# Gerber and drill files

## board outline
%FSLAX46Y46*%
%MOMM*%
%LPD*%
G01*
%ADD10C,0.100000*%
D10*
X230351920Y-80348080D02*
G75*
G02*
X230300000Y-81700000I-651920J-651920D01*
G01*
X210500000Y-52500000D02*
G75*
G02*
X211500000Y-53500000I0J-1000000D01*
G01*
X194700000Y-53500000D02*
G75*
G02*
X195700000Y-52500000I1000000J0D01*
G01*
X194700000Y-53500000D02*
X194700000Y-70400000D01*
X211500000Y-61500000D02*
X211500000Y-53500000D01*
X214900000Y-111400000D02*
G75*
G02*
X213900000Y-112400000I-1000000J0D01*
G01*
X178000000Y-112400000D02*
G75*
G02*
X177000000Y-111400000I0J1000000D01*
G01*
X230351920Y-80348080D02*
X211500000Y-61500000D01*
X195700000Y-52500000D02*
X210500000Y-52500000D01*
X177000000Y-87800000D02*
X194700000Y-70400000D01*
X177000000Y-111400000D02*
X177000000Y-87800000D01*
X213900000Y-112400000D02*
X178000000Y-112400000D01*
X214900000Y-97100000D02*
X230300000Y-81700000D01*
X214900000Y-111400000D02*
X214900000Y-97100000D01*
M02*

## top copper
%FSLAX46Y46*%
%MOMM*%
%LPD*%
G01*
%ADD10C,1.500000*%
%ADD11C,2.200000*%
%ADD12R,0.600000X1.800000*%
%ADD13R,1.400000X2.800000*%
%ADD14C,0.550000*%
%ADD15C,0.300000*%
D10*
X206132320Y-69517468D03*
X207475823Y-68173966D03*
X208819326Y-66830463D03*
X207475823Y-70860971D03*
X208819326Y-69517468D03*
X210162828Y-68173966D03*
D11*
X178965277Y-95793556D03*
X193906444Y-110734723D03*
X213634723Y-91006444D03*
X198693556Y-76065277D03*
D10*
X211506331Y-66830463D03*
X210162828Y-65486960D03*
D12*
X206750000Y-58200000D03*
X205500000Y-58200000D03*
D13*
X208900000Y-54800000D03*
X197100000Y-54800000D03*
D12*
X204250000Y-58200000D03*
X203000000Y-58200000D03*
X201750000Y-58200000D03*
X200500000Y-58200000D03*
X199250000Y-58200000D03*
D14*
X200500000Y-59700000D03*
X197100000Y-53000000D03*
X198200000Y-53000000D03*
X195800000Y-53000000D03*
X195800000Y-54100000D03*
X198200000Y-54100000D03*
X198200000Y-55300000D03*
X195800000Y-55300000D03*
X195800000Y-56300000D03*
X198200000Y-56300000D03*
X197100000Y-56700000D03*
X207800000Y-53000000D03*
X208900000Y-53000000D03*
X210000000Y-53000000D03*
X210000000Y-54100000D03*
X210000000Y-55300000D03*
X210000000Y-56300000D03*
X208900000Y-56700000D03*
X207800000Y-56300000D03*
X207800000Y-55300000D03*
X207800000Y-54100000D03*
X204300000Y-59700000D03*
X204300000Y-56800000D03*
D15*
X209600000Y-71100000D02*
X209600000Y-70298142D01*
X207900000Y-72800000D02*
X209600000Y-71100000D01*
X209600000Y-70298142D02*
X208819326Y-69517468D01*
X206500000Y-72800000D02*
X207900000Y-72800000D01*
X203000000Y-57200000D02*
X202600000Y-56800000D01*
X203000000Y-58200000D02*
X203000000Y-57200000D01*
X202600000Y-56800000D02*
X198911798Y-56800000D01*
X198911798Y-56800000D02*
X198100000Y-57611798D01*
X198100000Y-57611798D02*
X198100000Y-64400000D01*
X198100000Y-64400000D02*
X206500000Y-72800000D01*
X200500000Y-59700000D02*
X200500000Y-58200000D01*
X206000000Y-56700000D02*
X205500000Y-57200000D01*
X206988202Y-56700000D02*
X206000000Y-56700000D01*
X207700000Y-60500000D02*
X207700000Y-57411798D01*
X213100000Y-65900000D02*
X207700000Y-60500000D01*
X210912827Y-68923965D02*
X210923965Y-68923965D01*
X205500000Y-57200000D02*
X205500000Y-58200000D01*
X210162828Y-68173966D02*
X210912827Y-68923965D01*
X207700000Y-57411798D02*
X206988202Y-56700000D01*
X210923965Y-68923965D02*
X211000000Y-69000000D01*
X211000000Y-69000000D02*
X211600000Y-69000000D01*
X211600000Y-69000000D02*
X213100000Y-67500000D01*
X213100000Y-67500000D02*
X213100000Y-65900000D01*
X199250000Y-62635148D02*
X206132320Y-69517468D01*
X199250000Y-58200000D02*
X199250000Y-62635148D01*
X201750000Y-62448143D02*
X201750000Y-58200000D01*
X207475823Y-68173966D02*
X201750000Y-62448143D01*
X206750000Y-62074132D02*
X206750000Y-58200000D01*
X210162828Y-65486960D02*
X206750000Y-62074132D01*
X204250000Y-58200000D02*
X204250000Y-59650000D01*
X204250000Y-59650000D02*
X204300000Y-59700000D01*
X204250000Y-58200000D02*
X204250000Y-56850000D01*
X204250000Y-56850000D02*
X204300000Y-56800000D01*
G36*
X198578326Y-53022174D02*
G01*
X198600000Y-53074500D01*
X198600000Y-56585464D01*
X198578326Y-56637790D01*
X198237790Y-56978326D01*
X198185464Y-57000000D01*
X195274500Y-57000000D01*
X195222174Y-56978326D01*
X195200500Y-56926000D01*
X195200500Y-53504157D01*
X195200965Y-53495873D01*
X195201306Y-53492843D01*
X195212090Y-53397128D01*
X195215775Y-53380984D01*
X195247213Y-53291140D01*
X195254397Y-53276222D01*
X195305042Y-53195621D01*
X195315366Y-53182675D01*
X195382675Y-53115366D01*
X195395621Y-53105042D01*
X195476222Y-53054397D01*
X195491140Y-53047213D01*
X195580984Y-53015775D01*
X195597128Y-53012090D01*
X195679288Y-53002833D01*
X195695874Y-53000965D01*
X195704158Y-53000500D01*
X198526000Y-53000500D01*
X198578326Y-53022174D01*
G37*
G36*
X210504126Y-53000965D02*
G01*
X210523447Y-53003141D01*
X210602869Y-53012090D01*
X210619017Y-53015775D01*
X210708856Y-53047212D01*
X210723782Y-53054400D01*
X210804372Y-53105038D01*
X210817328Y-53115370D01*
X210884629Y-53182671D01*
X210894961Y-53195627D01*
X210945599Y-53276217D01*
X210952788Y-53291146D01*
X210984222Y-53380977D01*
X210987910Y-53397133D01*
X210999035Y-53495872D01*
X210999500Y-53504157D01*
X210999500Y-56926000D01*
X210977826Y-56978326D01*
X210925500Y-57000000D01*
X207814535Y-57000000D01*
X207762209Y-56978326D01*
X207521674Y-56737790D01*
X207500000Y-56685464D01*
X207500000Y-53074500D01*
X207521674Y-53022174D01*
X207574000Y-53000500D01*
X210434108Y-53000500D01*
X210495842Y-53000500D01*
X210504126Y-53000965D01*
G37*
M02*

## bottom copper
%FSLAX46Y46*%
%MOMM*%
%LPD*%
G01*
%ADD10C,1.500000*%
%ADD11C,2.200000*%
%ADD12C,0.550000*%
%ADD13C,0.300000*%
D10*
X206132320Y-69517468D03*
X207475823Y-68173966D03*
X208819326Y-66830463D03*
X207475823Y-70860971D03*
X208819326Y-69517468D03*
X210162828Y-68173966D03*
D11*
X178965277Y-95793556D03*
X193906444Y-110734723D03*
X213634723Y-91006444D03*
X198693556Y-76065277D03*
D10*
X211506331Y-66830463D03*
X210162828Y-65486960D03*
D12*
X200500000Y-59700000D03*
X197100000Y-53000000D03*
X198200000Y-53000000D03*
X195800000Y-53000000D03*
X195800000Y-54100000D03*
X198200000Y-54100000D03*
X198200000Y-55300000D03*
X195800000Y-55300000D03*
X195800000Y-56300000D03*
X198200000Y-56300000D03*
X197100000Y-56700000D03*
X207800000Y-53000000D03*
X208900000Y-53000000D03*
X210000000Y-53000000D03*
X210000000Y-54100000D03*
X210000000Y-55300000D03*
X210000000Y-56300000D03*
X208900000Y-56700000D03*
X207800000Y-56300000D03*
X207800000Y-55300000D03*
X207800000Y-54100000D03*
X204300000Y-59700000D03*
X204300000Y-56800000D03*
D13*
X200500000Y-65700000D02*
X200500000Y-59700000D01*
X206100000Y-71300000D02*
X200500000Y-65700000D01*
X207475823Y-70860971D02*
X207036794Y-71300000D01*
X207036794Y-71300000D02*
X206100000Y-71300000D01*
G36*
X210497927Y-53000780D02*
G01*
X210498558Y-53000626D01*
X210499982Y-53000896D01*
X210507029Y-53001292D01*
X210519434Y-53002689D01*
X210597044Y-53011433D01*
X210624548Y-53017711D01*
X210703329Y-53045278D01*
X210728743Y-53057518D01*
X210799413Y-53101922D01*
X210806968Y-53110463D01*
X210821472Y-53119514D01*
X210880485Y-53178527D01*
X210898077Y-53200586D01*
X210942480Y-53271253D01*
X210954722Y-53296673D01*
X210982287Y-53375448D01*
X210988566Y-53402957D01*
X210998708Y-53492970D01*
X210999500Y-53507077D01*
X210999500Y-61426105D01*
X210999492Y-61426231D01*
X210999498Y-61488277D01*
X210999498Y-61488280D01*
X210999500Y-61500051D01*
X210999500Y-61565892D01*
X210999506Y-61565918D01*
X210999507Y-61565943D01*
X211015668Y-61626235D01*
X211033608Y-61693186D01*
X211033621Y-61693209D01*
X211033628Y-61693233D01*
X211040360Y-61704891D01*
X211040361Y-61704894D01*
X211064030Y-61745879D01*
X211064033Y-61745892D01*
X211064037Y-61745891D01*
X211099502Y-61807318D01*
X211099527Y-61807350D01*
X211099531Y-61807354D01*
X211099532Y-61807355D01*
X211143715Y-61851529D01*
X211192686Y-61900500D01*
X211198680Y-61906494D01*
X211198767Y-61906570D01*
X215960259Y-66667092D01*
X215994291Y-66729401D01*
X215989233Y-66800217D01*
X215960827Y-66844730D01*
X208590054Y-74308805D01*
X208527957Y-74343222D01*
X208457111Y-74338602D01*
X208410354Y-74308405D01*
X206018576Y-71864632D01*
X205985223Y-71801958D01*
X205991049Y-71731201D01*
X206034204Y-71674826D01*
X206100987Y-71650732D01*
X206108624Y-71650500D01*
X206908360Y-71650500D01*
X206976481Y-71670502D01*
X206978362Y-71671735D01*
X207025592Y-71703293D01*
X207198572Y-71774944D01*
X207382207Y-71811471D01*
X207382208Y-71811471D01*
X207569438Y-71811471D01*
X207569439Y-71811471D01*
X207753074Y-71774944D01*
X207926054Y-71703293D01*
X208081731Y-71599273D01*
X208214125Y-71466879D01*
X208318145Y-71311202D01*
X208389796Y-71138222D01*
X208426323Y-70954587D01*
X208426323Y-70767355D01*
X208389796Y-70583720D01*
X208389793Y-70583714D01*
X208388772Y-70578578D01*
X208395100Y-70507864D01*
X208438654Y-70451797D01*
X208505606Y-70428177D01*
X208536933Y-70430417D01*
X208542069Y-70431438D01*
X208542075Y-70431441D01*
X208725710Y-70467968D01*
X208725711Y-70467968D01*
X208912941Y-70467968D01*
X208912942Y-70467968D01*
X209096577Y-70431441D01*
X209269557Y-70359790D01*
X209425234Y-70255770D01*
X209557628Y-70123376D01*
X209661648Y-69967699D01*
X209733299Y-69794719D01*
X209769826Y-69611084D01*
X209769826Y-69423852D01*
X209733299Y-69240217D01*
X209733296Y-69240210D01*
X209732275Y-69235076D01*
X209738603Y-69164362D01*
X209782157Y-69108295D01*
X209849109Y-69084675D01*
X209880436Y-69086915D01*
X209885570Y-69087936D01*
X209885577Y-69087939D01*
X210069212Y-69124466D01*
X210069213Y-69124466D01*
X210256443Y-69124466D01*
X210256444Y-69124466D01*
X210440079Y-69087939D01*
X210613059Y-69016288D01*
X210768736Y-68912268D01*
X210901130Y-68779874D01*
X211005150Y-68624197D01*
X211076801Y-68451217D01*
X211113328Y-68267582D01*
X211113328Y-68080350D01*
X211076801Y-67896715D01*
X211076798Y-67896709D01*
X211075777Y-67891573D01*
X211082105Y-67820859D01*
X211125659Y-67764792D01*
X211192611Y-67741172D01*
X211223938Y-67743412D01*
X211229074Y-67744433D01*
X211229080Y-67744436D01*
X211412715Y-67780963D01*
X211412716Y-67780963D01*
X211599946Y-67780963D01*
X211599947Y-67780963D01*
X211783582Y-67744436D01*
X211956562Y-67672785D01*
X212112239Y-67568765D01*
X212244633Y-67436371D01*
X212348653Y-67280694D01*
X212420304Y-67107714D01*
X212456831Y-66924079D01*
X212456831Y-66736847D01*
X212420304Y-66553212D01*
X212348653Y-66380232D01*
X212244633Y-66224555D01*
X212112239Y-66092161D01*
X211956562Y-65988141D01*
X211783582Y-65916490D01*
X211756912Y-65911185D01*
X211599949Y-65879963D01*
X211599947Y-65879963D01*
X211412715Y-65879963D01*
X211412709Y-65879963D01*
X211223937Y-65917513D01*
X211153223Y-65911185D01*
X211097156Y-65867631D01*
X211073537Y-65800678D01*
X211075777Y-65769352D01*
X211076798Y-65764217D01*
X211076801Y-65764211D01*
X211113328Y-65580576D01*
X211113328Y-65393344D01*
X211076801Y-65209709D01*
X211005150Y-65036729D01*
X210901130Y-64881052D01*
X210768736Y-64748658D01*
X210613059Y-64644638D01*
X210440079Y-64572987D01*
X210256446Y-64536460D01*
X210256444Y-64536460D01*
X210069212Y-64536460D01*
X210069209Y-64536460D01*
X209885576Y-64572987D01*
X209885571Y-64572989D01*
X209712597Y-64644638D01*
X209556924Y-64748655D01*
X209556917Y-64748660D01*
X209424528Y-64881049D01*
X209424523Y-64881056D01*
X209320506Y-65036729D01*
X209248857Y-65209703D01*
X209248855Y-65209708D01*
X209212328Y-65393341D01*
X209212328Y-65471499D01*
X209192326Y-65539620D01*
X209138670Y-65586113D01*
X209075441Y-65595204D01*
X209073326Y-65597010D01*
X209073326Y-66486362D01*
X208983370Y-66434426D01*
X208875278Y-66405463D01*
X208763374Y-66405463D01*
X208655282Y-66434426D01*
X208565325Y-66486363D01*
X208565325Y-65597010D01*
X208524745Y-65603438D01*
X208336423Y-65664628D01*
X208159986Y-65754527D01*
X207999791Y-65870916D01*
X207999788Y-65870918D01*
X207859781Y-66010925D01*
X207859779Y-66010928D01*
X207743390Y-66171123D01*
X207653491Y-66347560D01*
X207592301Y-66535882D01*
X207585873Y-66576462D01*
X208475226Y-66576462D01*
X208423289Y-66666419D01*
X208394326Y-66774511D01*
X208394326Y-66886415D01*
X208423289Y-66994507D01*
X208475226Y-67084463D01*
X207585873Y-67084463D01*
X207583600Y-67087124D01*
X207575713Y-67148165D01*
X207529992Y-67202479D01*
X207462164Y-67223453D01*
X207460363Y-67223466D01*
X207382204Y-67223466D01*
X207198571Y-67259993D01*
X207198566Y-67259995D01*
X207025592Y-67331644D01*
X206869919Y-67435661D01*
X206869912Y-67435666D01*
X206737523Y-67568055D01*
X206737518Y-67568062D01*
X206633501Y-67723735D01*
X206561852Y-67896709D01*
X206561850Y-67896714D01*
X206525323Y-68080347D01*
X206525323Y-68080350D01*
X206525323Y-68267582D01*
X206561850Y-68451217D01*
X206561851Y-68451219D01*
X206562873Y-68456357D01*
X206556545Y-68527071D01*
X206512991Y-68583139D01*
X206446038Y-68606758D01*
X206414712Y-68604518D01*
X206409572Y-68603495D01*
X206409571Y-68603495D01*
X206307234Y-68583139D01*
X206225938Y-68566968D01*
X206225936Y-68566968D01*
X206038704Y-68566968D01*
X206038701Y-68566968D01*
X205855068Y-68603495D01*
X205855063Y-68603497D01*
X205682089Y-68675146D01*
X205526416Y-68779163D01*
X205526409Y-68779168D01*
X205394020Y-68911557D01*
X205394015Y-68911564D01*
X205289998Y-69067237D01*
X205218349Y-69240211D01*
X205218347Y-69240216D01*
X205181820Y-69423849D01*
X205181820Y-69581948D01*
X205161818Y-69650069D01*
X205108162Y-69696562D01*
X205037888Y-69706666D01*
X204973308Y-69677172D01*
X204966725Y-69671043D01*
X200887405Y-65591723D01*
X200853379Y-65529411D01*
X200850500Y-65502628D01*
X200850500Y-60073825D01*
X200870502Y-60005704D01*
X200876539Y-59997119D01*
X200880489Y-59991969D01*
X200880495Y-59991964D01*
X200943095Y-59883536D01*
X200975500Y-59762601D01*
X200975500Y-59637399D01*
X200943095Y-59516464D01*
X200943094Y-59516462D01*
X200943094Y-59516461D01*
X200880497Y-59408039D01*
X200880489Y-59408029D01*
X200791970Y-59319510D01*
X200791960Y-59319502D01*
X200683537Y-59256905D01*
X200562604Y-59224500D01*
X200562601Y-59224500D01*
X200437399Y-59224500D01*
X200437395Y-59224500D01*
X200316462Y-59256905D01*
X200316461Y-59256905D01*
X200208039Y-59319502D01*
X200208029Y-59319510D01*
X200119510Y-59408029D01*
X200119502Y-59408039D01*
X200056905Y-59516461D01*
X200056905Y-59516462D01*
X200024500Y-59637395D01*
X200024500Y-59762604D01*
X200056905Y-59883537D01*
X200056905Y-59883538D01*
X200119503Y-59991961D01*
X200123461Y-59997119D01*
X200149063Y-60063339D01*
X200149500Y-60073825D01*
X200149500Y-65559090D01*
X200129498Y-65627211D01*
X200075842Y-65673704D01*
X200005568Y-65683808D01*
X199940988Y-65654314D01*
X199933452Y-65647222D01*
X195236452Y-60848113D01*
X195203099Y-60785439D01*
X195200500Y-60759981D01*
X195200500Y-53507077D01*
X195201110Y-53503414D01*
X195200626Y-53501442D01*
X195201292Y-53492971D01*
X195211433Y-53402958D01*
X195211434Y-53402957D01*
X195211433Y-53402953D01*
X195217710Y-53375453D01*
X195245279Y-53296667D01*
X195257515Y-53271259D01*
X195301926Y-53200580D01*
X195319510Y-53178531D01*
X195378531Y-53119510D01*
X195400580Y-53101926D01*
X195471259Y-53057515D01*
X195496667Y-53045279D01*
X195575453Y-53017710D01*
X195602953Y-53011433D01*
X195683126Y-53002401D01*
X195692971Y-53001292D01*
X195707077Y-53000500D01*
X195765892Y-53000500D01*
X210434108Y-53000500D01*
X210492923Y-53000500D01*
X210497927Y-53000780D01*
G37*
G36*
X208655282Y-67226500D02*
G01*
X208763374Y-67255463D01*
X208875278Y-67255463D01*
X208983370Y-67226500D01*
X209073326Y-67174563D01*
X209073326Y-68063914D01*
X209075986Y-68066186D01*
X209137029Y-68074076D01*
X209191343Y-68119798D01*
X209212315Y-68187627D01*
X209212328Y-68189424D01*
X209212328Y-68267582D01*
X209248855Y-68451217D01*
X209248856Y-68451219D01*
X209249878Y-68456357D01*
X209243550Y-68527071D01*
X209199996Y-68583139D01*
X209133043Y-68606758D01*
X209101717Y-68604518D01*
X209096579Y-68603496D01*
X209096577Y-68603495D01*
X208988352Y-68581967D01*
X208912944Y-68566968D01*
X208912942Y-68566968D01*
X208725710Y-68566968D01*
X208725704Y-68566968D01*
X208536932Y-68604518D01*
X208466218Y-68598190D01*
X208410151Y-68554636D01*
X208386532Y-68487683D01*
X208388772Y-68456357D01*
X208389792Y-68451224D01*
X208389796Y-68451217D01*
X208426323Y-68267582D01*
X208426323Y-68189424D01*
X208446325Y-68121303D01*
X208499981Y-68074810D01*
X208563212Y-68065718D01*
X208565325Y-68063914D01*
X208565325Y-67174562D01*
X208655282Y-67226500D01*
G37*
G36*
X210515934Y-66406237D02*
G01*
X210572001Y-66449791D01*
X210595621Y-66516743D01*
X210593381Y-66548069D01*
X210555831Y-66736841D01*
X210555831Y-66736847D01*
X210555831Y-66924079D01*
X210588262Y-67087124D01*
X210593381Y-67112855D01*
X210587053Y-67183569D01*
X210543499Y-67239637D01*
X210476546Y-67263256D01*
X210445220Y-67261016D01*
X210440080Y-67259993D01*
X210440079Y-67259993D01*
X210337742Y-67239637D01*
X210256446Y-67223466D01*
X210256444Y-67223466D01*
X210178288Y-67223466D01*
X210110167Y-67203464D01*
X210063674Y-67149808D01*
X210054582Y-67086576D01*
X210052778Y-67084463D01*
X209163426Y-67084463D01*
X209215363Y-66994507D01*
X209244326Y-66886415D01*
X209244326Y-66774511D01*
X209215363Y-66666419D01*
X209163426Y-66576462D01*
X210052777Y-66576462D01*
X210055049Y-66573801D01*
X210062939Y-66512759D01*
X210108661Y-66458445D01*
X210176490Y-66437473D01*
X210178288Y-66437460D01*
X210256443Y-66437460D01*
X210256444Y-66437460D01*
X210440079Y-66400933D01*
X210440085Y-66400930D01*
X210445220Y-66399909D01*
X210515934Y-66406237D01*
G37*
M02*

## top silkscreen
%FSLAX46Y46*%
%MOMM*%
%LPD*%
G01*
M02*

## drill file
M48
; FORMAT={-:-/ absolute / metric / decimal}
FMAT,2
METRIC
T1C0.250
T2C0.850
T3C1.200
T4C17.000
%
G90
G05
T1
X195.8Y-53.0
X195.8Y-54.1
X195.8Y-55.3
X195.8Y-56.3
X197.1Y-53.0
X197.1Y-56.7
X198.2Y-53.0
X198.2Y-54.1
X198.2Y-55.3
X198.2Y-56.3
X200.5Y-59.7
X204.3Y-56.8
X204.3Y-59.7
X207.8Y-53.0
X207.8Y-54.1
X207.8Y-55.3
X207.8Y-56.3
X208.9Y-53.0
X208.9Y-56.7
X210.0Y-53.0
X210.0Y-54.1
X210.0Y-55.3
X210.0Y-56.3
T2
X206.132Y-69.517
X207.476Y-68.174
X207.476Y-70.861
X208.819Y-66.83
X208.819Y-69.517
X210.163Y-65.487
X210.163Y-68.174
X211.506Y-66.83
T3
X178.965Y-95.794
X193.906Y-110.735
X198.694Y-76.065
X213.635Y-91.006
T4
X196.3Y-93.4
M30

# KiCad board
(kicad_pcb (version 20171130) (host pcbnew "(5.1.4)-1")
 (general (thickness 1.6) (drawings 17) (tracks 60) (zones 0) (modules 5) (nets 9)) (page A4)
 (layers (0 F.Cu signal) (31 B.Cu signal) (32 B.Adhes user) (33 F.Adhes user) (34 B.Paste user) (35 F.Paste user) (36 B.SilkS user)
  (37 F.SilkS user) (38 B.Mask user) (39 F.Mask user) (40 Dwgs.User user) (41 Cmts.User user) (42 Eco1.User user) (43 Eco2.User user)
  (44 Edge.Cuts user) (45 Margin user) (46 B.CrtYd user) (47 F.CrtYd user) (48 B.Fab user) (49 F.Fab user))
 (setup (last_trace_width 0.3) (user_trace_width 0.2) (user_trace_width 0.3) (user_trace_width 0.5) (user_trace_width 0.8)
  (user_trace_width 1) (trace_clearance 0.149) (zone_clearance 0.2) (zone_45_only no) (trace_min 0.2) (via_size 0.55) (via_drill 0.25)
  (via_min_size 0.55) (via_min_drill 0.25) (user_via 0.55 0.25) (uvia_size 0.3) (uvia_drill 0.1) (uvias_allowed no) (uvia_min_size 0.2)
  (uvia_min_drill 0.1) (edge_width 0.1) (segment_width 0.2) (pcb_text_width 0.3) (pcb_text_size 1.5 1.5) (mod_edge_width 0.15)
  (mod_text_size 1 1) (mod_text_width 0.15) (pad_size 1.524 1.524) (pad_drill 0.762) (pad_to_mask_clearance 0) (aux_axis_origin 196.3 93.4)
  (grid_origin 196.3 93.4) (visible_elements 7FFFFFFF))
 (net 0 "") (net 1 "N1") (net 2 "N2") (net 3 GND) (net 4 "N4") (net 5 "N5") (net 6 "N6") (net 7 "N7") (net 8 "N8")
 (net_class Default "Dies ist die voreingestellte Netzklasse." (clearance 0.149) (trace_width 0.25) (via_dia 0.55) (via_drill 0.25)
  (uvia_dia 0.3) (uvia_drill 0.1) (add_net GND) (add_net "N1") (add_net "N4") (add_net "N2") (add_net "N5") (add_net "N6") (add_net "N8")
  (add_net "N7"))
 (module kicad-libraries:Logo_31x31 (layer B.Cu) (at 207.7 105.8 180)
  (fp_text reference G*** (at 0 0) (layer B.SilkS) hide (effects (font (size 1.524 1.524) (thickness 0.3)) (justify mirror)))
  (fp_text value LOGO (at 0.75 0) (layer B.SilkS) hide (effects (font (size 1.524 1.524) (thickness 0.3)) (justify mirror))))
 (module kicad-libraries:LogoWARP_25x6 (layer B.Cu) (at 213.6 81 180)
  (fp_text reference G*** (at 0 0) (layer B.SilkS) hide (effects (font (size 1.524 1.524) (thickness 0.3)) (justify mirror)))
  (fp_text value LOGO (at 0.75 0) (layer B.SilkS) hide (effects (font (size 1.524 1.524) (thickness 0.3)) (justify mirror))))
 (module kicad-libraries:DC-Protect (layer F.Cu) (at 196.3 93.4 135)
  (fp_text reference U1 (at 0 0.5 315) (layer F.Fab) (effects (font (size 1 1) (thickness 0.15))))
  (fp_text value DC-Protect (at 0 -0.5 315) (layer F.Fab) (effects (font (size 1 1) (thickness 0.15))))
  (pad 1 thru_hole circle (at 9.935 23.84 135) (size 1.5 1.5) (drill 0.85) (layers *.Cu *.Mask) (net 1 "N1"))
  (pad 3 thru_hole circle (at 9.935 25.74 135) (size 1.5 1.5) (drill 0.85) (layers *.Cu *.Mask) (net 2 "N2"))
  (pad 5 thru_hole circle (at 9.935 27.64 135) (size 1.5 1.5) (drill 0.85) (layers *.Cu *.Mask) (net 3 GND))
  (pad 2 thru_hole circle (at 8.035 23.84 135) (size 1.5 1.5) (drill 0.85) (layers *.Cu *.Mask) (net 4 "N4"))
  (pad 4 thru_hole circle (at 8.035 25.74 135) (size 1.5 1.5) (drill 0.85) (layers *.Cu *.Mask) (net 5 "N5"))
  (pad 6 thru_hole circle (at 8.035 27.64 135) (size 1.5 1.5) (drill 0.85) (layers *.Cu *.Mask) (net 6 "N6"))
  (pad "" np_thru_hole circle (at 0 0 135) (size 17 17) (drill 17) (layers *.Cu *.Mask))
  (pad "" thru_hole circle (at 10.565 -13.95 135) (size 2.2 2.2) (drill 1.2) (layers *.Cu *.Mask))
  (pad "" thru_hole circle (at -10.565 -13.95 135) (size 2.2 2.2) (drill 1.2) (layers *.Cu *.Mask))
  (pad "" thru_hole circle (at -10.565 13.95 135) (size 2.2 2.2) (drill 1.2) (layers *.Cu *.Mask))
  (pad "" thru_hole circle (at 10.565 13.95 135) (size 2.2 2.2) (drill 1.2) (layers *.Cu *.Mask))
  (pad 8 thru_hole circle (at 8.035 29.54 135) (size 1.5 1.5) (drill 0.85) (layers *.Cu *.Mask) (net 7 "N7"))
  (pad 7 thru_hole circle (at 9.935 29.54 135) (size 1.5 1.5) (drill 0.85) (layers *.Cu *.Mask) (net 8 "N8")))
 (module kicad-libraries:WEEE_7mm (layer B.Cu) (at 181.2 107.1 180)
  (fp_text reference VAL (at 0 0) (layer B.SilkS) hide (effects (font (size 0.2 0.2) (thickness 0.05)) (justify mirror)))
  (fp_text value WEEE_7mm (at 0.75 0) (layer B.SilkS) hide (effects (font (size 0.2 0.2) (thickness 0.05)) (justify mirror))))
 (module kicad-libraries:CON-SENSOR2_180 (layer F.Cu) (at 203 53.4 180)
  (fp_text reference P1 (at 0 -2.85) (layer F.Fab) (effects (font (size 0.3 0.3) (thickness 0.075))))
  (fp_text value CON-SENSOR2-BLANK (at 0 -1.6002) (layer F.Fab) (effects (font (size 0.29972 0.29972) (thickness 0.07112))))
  (pad 7 smd rect (at -3.75 -4.8 180) (size 0.6 1.8) (layers F.Cu F.Paste F.Mask) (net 8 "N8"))
  (pad 6 smd rect (at -2.5 -4.8 180) (size 0.6 1.8) (layers F.Cu F.Paste F.Mask) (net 6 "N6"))
  (pad EP smd rect (at -5.9 -1.4 180) (size 1.4 2.8) (layers F.Cu F.Paste F.Mask) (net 3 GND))
  (pad EP smd rect (at 5.9 -1.4 180) (size 1.4 2.8) (layers F.Cu F.Paste F.Mask) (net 3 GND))
  (pad 5 smd rect (at -1.25 -4.8 180) (size 0.6 1.8) (layers F.Cu F.Paste F.Mask) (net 3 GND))
  (pad 4 smd rect (at 0 -4.8 180) (size 0.6 1.8) (layers F.Cu F.Paste F.Mask) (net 5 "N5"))
  (pad 3 smd rect (at 1.25 -4.8 180) (size 0.6 1.8) (layers F.Cu F.Paste F.Mask) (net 2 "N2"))
  (pad 2 smd rect (at 2.5 -4.8 180) (size 0.6 1.8) (layers F.Cu F.Paste F.Mask) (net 4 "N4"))
  (pad 1 smd rect (at 3.75 -4.8 180) (size 0.6 1.8) (layers F.Cu F.Paste F.Mask) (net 1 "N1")))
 (gr_arc (start 229.7 81) (end 230.3 81.7) (angle -94.39870535) (layer Edge.Cuts) (width 0.1))
 (gr_arc (start 210.5 53.5) (end 211.5 53.5) (angle -90) (layer Edge.Cuts) (width 0.1))
 (gr_arc (start 195.7 53.5) (end 195.7 52.5) (angle -90) (layer Edge.Cuts) (width 0.1))
 (gr_line (start 194.7 53.5) (end 194.7 70.4) (layer Edge.Cuts) (width 0.1))
 (gr_line (start 211.5 61.5) (end 211.5 53.5) (layer Edge.Cuts) (width 0.1))
 (gr_arc (start 213.9 111.4) (end 213.9 112.4) (angle -90) (layer Edge.Cuts) (width 0.1))
 (gr_arc (start 178 111.4) (end 177 111.4) (angle -90) (layer Edge.Cuts) (width 0.1))
 (gr_line (start 230.35192 80.34808) (end 211.5 61.5) (layer Edge.Cuts) (width 0.1))
 (gr_line (start 195.7 52.5) (end 210.5 52.5) (layer Edge.Cuts) (width 0.1))
 (gr_line (start 177 87.8) (end 194.7 70.4) (layer Edge.Cuts) (width 0.1))
 (gr_line (start 177 111.4) (end 177 87.8) (layer Edge.Cuts) (width 0.1))
 (gr_line (start 213.9 112.4) (end 178 112.4) (layer Edge.Cuts) (width 0.1))
 (gr_line (start 214.9 97.1) (end 230.3 81.7) (layer Edge.Cuts) (width 0.1))
 (gr_line (start 214.9 111.4) (end 214.9 97.1) (layer Edge.Cuts) (width 0.1))
 (segment (start 209.6 71.1) (end 209.6 70.298142) (width 0.3) (layer F.Cu) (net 5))
 (segment (start 207.9 72.8) (end 209.6 71.1) (width 0.3) (layer F.Cu) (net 5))
 (segment (start 209.6 70.298142) (end 208.819326 69.517468) (width 0.3) (layer F.Cu) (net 5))
 (segment (start 206.5 72.8) (end 207.9 72.8) (width 0.3) (layer F.Cu) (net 5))
 (segment (start 203 57.2) (end 202.6 56.8) (width 0.3) (layer F.Cu) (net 5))
 (segment (start 203 58.2) (end 203 57.2) (width 0.3) (layer F.Cu) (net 5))
 (segment (start 202.6 56.8) (end 198.911798 56.8) (width 0.3) (layer F.Cu) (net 5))
 (segment (start 198.911798 56.8) (end 198.1 57.611798) (width 0.3) (layer F.Cu) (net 5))
 (segment (start 198.1 57.611798) (end 198.1 64.4) (width 0.3) (layer F.Cu) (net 5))
 (segment (start 198.1 64.4) (end 206.5 72.8) (width 0.3) (layer F.Cu) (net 5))
 (via (at 200.5 59.7) (size 0.55) (drill 0.25) (layers F.Cu B.Cu) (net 4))
 (segment (start 200.5 59.7) (end 200.5 58.2) (width 0.3) (layer F.Cu) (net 4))
 (segment (start 200.5 65.7) (end 200.5 59.7) (width 0.3) (layer B.Cu) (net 4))
 (segment (start 206.1 71.3) (end 200.5 65.7) (width 0.3) (layer B.Cu) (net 4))
 (segment (start 207.475823 70.860971) (end 207.036794 71.3) (width 0.3) (layer B.Cu) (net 4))
 (segment (start 207.036794 71.3) (end 206.1 71.3) (width 0.3) (layer B.Cu) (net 4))
 (segment (start 206 56.7) (end 205.5 57.2) (width 0.3) (layer F.Cu) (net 6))
 (segment (start 206.988202 56.7) (end 206 56.7) (width 0.3) (layer F.Cu) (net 6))
 (segment (start 207.7 60.5) (end 207.7 57.411798) (width 0.3) (layer F.Cu) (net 6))
 (segment (start 213.1 65.9) (end 207.7 60.5) (width 0.3) (layer F.Cu) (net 6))
 (segment (start 210.912827 68.923965) (end 210.923965 68.923965) (width 0.3) (layer F.Cu) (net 6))
 (segment (start 205.5 57.2) (end 205.5 58.2) (width 0.3) (layer F.Cu) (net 6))
 (segment (start 210.162828 68.173966) (end 210.912827 68.923965) (width 0.3) (layer F.Cu) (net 6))
 (segment (start 207.7 57.411798) (end 206.988202 56.7) (width 0.3) (layer F.Cu) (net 6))
 (segment (start 210.923965 68.923965) (end 211 69) (width 0.3) (layer F.Cu) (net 6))
 (segment (start 211 69) (end 211.6 69) (width 0.3) (layer F.Cu) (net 6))
 (segment (start 211.6 69) (end 213.1 67.5) (width 0.3) (layer F.Cu) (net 6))
 (segment (start 213.1 67.5) (end 213.1 65.9) (width 0.3) (layer F.Cu) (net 6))
 (segment (start 199.25 62.635148) (end 206.13232 69.517468) (width 0.3) (layer F.Cu) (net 1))
 (segment (start 199.25 58.2) (end 199.25 62.635148) (width 0.3) (layer F.Cu) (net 1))
 (segment (start 201.75 62.448143) (end 201.75 58.2) (width 0.3) (layer F.Cu) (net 2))
 (segment (start 207.475823 68.173966) (end 201.75 62.448143) (width 0.3) (layer F.Cu) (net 2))
 (segment (start 206.75 62.074132) (end 206.75 58.2) (width 0.3) (layer F.Cu) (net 8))
 (segment (start 210.162828 65.48696) (end 206.75 62.074132) (width 0.3) (layer F.Cu) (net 8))
 (via (at 197.1 53) (size 0.55) (drill 0.25) (layers F.Cu B.Cu) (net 3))
 (via (at 198.2 53) (size 0.55) (drill 0.25) (layers F.Cu B.Cu) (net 3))
 (via (at 195.8 53) (size 0.55) (drill 0.25) (layers F.Cu B.Cu) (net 3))
 (via (at 195.8 54.1) (size 0.55) (drill 0.25) (layers F.Cu B.Cu) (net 3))
 (via (at 198.2 54.1) (size 0.55) (drill 0.25) (layers F.Cu B.Cu) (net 3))
 (via (at 198.2 55.3) (size 0.55) (drill 0.25) (layers F.Cu B.Cu) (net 3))
 (via (at 195.8 55.3) (size 0.55) (drill 0.25) (layers F.Cu B.Cu) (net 3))
 (via (at 195.8 56.3) (size 0.55) (drill 0.25) (layers F.Cu B.Cu) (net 3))
 (via (at 198.2 56.3) (size 0.55) (drill 0.25) (layers F.Cu B.Cu) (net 3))
 (via (at 197.1 56.7) (size 0.55) (drill 0.25) (layers F.Cu B.Cu) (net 3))
 (via (at 207.8 53) (size 0.55) (drill 0.25) (layers F.Cu B.Cu) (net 3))
 (via (at 208.9 53) (size 0.55) (drill 0.25) (layers F.Cu B.Cu) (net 3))
 (via (at 210 53) (size 0.55) (drill 0.25) (layers F.Cu B.Cu) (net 3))
 (via (at 210 54.1) (size 0.55) (drill 0.25) (layers F.Cu B.Cu) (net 3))
 (via (at 210 55.3) (size 0.55) (drill 0.25) (layers F.Cu B.Cu) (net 3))
 (via (at 210 56.3) (size 0.55) (drill 0.25) (layers F.Cu B.Cu) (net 3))
 (via (at 208.9 56.7) (size 0.55) (drill 0.25) (layers F.Cu B.Cu) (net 3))
 (via (at 207.8 56.3) (size 0.55) (drill 0.25) (layers F.Cu B.Cu) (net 3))
 (via (at 207.8 55.3) (size 0.55) (drill 0.25) (layers F.Cu B.Cu) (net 3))
 (via (at 207.8 54.1) (size 0.55) (drill 0.25) (layers F.Cu B.Cu) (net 3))
 (via (at 204.3 59.7) (size 0.55) (drill 0.25) (layers F.Cu B.Cu) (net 3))
 (segment (start 204.25 58.2) (end 204.25 59.65) (width 0.3) (layer F.Cu) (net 3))
 (segment (start 204.25 59.65) (end 204.3 59.7) (width 0.3) (layer F.Cu) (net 3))
 (via (at 204.3 56.8) (size 0.55) (drill 0.25) (layers F.Cu B.Cu) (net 3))
 (segment (start 204.25 58.2) (end 204.25 56.85) (width 0.3) (layer F.Cu) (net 3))
 (segment (start 204.25 56.85) (end 204.3 56.8) (width 0.3) (layer F.Cu) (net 3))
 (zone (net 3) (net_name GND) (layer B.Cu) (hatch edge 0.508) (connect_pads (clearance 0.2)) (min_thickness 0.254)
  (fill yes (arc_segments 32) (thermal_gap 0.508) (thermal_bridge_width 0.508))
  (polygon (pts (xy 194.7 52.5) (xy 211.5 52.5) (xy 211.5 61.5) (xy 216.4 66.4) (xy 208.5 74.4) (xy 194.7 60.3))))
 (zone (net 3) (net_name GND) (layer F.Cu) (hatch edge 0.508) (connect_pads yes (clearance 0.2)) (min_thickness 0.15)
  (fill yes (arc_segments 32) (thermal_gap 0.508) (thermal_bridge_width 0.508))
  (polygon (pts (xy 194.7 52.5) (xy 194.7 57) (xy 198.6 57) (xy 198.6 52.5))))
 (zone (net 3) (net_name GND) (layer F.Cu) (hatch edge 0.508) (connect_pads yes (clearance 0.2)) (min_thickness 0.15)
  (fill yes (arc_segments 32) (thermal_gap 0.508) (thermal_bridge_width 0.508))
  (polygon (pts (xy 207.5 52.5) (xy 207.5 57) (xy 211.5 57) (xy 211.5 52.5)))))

